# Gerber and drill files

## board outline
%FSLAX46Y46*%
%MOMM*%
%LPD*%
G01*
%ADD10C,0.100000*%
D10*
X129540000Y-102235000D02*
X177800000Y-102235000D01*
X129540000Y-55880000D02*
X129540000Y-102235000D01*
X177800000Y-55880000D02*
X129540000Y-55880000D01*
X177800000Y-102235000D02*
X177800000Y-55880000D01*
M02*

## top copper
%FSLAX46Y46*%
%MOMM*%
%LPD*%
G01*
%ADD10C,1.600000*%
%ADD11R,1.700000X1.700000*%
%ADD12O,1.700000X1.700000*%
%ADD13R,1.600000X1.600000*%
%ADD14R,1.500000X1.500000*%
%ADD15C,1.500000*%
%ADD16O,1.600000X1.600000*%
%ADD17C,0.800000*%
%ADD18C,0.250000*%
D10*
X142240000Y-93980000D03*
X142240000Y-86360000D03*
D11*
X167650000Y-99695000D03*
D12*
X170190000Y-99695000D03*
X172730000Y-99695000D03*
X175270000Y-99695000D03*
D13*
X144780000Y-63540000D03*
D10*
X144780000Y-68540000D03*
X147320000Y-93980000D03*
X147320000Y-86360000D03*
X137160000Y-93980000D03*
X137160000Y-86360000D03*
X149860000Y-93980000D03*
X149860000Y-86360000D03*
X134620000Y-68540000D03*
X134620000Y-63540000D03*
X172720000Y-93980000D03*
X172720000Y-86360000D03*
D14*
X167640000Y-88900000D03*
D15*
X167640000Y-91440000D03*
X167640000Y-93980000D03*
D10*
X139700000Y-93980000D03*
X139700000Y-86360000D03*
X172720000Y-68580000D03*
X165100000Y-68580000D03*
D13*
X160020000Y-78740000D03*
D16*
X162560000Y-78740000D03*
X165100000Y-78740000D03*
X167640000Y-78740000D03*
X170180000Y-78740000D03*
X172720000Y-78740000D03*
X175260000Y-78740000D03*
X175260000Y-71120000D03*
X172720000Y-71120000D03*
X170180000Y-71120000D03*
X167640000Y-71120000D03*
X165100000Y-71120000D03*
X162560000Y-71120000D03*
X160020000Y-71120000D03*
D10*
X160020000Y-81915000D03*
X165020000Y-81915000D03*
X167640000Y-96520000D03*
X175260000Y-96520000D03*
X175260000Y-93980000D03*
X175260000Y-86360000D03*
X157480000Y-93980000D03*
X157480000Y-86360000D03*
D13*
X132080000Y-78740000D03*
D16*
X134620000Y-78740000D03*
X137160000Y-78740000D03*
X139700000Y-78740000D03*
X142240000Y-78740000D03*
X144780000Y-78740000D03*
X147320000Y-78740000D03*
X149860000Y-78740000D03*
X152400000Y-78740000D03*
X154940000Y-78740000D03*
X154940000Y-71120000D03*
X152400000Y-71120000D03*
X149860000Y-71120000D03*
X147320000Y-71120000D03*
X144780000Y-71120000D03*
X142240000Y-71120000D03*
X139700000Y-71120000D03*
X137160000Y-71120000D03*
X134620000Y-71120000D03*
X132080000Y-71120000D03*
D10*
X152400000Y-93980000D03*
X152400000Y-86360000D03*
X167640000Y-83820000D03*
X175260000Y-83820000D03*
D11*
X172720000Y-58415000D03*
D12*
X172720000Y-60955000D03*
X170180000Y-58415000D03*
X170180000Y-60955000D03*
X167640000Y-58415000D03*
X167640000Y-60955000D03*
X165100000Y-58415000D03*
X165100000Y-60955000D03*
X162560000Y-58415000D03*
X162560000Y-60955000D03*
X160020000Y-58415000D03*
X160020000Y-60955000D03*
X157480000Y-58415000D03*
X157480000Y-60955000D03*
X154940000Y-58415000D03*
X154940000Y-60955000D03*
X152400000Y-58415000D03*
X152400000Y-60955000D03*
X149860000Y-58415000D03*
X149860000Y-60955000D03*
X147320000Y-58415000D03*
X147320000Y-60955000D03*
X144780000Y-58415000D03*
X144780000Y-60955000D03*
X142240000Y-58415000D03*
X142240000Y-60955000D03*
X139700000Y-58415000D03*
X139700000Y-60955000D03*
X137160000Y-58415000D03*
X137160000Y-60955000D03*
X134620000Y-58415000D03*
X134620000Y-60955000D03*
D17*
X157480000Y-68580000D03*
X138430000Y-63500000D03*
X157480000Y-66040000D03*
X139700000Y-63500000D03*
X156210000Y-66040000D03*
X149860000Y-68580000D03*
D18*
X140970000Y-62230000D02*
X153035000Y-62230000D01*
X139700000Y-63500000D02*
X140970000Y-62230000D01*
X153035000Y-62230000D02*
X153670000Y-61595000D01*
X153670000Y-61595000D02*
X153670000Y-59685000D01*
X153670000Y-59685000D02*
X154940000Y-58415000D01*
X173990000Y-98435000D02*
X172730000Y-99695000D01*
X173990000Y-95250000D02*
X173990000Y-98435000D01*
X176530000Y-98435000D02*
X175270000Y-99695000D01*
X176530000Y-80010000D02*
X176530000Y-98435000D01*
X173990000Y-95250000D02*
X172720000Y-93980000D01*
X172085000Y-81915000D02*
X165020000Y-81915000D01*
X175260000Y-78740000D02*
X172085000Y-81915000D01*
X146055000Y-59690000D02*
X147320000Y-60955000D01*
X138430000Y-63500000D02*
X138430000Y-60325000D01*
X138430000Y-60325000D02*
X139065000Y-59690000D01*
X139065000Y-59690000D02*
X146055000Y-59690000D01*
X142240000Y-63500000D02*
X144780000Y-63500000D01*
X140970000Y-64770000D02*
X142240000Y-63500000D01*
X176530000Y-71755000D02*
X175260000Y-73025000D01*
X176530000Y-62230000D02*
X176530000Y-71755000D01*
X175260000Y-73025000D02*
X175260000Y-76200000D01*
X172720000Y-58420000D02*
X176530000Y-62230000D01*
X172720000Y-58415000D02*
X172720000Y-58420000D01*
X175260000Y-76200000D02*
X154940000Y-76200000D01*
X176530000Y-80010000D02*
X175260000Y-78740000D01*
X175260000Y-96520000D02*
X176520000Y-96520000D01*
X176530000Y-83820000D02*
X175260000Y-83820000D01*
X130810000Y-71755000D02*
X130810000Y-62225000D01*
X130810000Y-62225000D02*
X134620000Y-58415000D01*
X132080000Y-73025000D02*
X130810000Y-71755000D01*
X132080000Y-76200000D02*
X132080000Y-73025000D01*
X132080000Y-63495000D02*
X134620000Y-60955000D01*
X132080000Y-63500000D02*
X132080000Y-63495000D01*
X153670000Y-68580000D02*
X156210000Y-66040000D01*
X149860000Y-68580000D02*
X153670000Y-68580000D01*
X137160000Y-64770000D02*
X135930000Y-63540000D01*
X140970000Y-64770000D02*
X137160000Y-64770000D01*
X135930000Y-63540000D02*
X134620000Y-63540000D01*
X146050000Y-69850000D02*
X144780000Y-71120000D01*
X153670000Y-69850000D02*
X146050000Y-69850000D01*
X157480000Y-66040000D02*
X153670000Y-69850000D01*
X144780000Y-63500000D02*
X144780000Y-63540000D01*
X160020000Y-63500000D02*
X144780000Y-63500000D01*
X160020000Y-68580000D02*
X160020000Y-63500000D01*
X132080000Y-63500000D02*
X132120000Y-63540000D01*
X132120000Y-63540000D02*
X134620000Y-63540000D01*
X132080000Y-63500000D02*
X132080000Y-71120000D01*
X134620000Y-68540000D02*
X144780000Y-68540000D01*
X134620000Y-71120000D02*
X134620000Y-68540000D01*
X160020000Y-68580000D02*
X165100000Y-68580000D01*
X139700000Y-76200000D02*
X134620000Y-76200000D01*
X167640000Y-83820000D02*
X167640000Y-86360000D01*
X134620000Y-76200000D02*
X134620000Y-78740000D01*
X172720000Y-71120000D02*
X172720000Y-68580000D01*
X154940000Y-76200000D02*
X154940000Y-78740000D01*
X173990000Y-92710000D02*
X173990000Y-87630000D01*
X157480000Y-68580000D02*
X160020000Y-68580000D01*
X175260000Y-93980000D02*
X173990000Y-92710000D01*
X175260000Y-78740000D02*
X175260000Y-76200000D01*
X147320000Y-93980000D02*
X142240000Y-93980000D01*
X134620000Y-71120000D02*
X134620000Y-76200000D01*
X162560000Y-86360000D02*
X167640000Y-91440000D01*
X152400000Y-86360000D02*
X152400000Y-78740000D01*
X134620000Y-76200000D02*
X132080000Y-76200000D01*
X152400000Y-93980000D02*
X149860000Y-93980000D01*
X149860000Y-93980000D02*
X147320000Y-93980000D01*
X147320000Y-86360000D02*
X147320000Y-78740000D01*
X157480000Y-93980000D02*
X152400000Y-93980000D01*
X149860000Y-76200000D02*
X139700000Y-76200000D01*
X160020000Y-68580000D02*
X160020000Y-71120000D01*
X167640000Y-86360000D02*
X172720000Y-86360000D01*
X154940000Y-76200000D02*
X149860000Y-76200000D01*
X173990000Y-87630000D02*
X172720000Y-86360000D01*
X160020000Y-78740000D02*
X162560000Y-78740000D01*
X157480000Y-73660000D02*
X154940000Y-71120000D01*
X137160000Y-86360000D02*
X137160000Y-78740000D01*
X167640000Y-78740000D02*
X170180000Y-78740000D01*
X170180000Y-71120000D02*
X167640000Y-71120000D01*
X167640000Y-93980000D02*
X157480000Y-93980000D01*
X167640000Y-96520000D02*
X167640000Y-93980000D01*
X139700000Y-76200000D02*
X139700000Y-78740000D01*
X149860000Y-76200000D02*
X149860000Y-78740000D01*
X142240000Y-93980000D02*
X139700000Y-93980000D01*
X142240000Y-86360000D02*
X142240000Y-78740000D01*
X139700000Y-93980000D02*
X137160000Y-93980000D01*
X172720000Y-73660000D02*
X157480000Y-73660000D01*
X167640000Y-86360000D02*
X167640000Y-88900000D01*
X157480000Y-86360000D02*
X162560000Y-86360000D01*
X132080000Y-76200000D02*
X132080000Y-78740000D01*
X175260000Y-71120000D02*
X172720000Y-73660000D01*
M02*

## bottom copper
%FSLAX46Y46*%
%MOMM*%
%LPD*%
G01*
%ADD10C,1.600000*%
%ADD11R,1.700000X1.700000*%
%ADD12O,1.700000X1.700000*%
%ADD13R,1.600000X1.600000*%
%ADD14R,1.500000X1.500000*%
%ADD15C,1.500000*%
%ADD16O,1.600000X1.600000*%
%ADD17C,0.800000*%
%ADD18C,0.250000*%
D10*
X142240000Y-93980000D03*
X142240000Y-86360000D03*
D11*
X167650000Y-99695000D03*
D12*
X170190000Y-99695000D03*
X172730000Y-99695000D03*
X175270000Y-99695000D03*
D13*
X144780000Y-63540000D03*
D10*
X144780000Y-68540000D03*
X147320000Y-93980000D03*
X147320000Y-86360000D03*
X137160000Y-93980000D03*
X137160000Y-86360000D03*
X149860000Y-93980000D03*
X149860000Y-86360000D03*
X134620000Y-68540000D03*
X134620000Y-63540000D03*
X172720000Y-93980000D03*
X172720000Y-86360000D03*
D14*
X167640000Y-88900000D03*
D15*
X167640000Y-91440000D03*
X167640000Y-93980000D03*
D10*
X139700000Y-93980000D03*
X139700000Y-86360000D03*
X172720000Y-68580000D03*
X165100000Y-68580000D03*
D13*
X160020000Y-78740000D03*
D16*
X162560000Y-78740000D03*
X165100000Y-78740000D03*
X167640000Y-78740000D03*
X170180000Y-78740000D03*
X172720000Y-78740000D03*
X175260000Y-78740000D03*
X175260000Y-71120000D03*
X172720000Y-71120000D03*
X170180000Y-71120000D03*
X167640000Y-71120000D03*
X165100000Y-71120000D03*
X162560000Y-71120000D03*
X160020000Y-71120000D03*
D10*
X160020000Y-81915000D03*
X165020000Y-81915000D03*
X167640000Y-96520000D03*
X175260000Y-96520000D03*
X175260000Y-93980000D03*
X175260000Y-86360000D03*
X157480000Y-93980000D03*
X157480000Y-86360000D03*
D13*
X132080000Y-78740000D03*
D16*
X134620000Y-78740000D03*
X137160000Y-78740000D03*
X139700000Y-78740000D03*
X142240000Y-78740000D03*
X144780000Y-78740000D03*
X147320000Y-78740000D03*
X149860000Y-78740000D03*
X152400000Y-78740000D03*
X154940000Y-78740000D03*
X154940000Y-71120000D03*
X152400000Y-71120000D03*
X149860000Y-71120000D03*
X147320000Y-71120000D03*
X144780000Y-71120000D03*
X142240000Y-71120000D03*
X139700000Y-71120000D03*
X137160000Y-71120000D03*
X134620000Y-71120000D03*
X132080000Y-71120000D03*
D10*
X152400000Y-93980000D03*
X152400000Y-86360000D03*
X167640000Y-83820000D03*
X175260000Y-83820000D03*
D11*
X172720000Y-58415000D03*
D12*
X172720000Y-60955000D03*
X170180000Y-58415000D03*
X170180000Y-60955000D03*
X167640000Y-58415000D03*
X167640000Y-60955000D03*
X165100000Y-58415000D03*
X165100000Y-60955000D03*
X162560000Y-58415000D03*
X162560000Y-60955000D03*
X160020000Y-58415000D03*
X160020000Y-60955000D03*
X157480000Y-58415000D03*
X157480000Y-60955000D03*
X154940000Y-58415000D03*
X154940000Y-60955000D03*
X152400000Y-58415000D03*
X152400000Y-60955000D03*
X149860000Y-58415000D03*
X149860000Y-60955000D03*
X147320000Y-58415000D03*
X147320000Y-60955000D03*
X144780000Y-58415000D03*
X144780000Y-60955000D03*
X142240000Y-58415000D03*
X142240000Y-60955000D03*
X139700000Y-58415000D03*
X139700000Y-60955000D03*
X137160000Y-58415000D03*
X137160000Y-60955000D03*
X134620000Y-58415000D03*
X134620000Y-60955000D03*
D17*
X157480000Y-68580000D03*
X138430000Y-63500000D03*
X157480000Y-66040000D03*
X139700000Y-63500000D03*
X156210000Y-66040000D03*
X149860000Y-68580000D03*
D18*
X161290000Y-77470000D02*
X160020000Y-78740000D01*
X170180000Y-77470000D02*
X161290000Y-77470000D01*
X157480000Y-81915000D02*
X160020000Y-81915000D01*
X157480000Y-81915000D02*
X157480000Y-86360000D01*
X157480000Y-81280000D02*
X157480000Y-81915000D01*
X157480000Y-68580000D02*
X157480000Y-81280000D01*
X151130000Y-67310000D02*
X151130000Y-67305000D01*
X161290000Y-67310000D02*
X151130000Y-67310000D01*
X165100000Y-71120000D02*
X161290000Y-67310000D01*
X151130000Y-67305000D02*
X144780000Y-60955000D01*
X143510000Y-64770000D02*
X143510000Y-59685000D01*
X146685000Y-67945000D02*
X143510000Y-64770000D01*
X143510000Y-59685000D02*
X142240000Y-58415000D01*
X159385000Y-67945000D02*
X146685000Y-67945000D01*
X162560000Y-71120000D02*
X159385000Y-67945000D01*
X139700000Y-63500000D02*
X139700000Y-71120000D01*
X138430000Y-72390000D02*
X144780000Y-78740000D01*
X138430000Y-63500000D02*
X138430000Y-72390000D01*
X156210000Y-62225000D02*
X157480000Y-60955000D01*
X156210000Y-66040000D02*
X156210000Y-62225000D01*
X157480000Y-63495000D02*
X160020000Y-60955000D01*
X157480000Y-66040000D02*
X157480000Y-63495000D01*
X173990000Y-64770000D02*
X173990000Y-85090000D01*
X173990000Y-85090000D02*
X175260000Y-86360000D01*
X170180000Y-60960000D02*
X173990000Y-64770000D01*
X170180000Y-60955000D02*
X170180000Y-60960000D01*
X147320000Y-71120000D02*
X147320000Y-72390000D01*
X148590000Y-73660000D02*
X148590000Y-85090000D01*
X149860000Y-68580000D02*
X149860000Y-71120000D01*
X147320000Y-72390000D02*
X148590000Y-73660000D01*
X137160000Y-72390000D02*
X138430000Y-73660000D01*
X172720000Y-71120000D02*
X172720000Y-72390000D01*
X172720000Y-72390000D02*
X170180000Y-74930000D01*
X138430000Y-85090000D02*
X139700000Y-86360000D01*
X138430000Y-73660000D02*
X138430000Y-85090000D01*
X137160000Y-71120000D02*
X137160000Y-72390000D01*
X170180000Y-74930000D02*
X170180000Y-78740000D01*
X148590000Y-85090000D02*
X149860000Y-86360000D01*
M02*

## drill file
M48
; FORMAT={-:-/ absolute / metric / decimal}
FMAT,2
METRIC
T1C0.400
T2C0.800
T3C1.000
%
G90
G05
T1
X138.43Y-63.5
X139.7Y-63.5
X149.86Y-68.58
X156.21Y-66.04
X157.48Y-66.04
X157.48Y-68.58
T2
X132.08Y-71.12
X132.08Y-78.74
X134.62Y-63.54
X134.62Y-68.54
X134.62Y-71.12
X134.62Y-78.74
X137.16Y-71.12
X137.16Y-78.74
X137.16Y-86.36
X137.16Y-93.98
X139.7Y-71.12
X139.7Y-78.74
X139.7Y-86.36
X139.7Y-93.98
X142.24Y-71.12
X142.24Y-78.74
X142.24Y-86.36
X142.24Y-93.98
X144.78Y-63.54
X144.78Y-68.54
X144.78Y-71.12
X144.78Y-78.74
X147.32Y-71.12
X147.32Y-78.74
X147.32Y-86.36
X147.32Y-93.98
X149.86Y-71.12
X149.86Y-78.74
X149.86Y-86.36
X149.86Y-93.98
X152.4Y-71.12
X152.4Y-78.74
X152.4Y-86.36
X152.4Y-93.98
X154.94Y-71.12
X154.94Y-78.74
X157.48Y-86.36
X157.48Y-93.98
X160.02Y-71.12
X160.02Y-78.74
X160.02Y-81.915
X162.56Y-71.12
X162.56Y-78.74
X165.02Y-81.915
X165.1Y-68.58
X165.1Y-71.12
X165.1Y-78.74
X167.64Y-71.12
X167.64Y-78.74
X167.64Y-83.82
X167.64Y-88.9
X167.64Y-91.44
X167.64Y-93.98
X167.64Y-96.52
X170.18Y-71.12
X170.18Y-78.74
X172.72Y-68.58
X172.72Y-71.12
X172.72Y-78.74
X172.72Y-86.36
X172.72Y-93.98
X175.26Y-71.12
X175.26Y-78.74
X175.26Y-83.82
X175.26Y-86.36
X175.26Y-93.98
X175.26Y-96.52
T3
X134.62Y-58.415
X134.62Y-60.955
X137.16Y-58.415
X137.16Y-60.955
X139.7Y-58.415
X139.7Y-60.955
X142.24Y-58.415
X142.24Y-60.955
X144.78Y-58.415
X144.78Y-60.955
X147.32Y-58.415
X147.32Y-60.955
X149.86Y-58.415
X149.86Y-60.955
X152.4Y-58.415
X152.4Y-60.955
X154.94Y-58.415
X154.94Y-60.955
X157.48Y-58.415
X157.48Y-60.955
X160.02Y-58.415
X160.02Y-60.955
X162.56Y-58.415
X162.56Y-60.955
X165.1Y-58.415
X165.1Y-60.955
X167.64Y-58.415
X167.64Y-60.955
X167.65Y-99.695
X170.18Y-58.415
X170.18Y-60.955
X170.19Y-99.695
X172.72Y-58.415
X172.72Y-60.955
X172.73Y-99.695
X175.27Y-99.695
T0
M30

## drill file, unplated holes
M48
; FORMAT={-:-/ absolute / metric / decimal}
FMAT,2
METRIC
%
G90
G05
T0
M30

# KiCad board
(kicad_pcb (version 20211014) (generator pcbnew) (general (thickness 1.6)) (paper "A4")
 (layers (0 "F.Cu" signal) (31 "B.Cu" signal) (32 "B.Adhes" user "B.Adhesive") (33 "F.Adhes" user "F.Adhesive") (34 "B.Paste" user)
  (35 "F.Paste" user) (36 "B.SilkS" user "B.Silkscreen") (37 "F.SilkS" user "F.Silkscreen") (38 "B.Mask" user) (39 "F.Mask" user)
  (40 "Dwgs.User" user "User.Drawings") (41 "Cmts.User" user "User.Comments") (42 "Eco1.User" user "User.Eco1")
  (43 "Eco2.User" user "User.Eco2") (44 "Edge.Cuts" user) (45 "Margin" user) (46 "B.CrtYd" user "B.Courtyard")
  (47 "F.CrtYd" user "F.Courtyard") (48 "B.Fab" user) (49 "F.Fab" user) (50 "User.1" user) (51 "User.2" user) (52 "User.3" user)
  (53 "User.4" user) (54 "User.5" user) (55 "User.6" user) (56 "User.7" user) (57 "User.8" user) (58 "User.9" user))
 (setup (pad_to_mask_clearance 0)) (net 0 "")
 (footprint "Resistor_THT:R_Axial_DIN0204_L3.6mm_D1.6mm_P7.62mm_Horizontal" (layer "F.Cu") (at 142.24 93.98 90)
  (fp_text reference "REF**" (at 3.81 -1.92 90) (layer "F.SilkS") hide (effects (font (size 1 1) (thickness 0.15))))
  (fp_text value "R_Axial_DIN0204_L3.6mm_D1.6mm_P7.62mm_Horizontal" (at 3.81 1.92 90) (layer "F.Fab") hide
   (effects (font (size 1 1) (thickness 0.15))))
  (pad "1" thru_hole circle (at 0 0 90) (size 1.6 1.6) (drill 0.8) (layers *.Cu *.Mask))
  (pad "2" thru_hole circle (at 7.62 0 90) (size 1.6 1.6) (drill 0.8) (layers *.Cu *.Mask)))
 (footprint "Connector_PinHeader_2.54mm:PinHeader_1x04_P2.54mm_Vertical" (layer "F.Cu") (at 167.65 99.695 90)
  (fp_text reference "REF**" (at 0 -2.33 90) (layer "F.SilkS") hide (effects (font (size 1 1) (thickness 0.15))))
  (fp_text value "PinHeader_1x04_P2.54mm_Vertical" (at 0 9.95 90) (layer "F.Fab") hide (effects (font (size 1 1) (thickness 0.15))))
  (pad "1" thru_hole rect (at 0 0 90) (size 1.7 1.7) (drill 1) (layers *.Cu *.Mask))
  (pad "2" thru_hole oval (at 0 2.54 90) (size 1.7 1.7) (drill 1) (layers *.Cu *.Mask))
  (pad "3" thru_hole oval (at 0 5.08 90) (size 1.7 1.7) (drill 1) (layers *.Cu *.Mask))
  (pad "4" thru_hole oval (at 0 7.62 90) (size 1.7 1.7) (drill 1) (layers *.Cu *.Mask)))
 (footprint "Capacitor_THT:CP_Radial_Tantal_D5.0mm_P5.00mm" (layer "F.Cu") (at 144.78 63.54 -90)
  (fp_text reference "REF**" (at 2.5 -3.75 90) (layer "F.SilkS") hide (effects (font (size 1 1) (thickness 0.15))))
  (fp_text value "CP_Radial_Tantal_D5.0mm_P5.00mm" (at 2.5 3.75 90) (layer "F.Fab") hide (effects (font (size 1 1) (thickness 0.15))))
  (pad "1" thru_hole rect (at 0 0 270) (size 1.6 1.6) (drill 0.8) (layers *.Cu *.Mask))
  (pad "2" thru_hole circle (at 5 0 270) (size 1.6 1.6) (drill 0.8) (layers *.Cu *.Mask)))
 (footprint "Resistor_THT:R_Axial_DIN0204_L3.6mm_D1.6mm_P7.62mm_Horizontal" (layer "F.Cu") (at 147.32 93.98 90)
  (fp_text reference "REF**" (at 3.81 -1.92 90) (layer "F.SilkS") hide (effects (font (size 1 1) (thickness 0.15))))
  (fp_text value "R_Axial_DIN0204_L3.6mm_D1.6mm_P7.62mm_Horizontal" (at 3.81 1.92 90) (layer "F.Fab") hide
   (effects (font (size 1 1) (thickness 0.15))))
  (pad "1" thru_hole circle (at 0 0 90) (size 1.6 1.6) (drill 0.8) (layers *.Cu *.Mask))
  (pad "2" thru_hole circle (at 7.62 0 90) (size 1.6 1.6) (drill 0.8) (layers *.Cu *.Mask)))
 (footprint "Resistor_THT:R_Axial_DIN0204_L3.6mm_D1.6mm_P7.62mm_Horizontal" (layer "F.Cu") (at 137.16 93.98 90)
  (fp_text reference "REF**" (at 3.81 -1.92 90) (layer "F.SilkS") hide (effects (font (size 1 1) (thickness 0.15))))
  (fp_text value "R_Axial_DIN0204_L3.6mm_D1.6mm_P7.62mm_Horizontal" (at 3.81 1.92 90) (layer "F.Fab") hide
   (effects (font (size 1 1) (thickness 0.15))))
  (pad "1" thru_hole circle (at 0 0 90) (size 1.6 1.6) (drill 0.8) (layers *.Cu *.Mask))
  (pad "2" thru_hole circle (at 7.62 0 90) (size 1.6 1.6) (drill 0.8) (layers *.Cu *.Mask)))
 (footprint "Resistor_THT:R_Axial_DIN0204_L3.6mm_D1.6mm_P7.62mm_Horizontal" (layer "F.Cu") (at 149.86 93.98 90)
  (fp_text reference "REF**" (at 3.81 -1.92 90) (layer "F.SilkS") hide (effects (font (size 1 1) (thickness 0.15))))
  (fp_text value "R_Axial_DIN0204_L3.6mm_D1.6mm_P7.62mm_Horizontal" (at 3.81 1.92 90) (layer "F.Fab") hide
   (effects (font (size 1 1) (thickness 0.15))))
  (pad "1" thru_hole circle (at 0 0 90) (size 1.6 1.6) (drill 0.8) (layers *.Cu *.Mask))
  (pad "2" thru_hole circle (at 7.62 0 90) (size 1.6 1.6) (drill 0.8) (layers *.Cu *.Mask)))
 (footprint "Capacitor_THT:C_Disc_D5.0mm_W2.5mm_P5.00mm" (layer "F.Cu") (at 134.62 68.54 90)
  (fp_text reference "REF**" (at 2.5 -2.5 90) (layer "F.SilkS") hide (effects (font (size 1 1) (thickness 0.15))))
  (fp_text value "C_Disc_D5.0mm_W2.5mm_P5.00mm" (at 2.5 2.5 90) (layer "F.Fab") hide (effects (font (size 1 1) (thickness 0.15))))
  (pad "1" thru_hole circle (at 0 0 90) (size 1.6 1.6) (drill 0.8) (layers *.Cu *.Mask))
  (pad "2" thru_hole circle (at 5 0 90) (size 1.6 1.6) (drill 0.8) (layers *.Cu *.Mask)))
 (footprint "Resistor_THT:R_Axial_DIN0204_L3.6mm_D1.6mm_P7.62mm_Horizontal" (layer "F.Cu") (at 172.72 93.98 90)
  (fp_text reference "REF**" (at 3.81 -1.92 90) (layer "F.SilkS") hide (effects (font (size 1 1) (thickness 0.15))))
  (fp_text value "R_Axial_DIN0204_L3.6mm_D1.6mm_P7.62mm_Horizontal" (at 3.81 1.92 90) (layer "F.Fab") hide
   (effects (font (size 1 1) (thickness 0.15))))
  (pad "1" thru_hole circle (at 0 0 90) (size 1.6 1.6) (drill 0.8) (layers *.Cu *.Mask))
  (pad "2" thru_hole circle (at 7.62 0 90) (size 1.6 1.6) (drill 0.8) (layers *.Cu *.Mask)))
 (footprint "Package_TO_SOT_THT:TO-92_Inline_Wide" (layer "F.Cu") (at 167.64 88.9 -90)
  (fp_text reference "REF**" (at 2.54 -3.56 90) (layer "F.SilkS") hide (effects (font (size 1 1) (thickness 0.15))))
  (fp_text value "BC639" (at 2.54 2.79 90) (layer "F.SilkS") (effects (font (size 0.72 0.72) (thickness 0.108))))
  (pad "1" thru_hole rect (at 0 0 270) (size 1.5 1.5) (drill 0.8) (layers *.Cu *.Mask))
  (pad "2" thru_hole circle (at 2.54 0 270) (size 1.5 1.5) (drill 0.8) (layers *.Cu *.Mask))
  (pad "3" thru_hole circle (at 5.08 0 270) (size 1.5 1.5) (drill 0.8) (layers *.Cu *.Mask)))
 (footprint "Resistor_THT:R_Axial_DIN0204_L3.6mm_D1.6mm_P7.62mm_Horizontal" (layer "F.Cu") (at 139.7 93.98 90)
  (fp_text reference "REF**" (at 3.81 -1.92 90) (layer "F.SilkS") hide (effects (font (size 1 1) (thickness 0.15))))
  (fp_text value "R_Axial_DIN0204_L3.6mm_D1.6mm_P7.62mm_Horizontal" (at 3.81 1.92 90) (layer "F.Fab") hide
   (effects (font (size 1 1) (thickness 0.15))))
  (pad "1" thru_hole circle (at 0 0 90) (size 1.6 1.6) (drill 0.8) (layers *.Cu *.Mask))
  (pad "2" thru_hole circle (at 7.62 0 90) (size 1.6 1.6) (drill 0.8) (layers *.Cu *.Mask)))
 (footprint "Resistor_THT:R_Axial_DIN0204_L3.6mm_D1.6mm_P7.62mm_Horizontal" (layer "F.Cu") (at 172.72 68.58 180)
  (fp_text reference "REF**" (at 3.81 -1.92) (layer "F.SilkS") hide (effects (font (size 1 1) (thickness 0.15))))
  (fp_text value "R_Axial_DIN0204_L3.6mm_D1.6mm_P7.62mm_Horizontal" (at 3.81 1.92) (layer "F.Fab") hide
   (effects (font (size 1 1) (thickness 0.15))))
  (pad "1" thru_hole circle (at 0 0 180) (size 1.6 1.6) (drill 0.8) (layers *.Cu *.Mask))
  (pad "2" thru_hole circle (at 7.62 0 180) (size 1.6 1.6) (drill 0.8) (layers *.Cu *.Mask)))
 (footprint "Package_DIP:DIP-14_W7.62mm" (layer "F.Cu") (at 160.02 78.74 90)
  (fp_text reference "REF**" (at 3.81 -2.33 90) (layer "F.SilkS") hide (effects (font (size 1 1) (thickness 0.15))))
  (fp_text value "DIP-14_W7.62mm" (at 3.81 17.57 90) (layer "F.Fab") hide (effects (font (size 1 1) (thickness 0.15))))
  (pad "1" thru_hole rect (at 0 0 90) (size 1.6 1.6) (drill 0.8) (layers *.Cu *.Mask))
  (pad "2" thru_hole oval (at 0 2.54 90) (size 1.6 1.6) (drill 0.8) (layers *.Cu *.Mask))
  (pad "3" thru_hole oval (at 0 5.08 90) (size 1.6 1.6) (drill 0.8) (layers *.Cu *.Mask))
  (pad "4" thru_hole oval (at 0 7.62 90) (size 1.6 1.6) (drill 0.8) (layers *.Cu *.Mask))
  (pad "5" thru_hole oval (at 0 10.16 90) (size 1.6 1.6) (drill 0.8) (layers *.Cu *.Mask))
  (pad "6" thru_hole oval (at 0 12.7 90) (size 1.6 1.6) (drill 0.8) (layers *.Cu *.Mask))
  (pad "7" thru_hole oval (at 0 15.24 90) (size 1.6 1.6) (drill 0.8) (layers *.Cu *.Mask))
  (pad "8" thru_hole oval (at 7.62 15.24 90) (size 1.6 1.6) (drill 0.8) (layers *.Cu *.Mask))
  (pad "9" thru_hole oval (at 7.62 12.7 90) (size 1.6 1.6) (drill 0.8) (layers *.Cu *.Mask))
  (pad "10" thru_hole oval (at 7.62 10.16 90) (size 1.6 1.6) (drill 0.8) (layers *.Cu *.Mask))
  (pad "11" thru_hole oval (at 7.62 7.62 90) (size 1.6 1.6) (drill 0.8) (layers *.Cu *.Mask))
  (pad "12" thru_hole oval (at 7.62 5.08 90) (size 1.6 1.6) (drill 0.8) (layers *.Cu *.Mask))
  (pad "13" thru_hole oval (at 7.62 2.54 90) (size 1.6 1.6) (drill 0.8) (layers *.Cu *.Mask))
  (pad "14" thru_hole oval (at 7.62 0 90) (size 1.6 1.6) (drill 0.8) (layers *.Cu *.Mask)))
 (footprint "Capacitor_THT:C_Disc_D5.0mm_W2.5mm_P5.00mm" (layer "F.Cu") (at 160.02 81.915)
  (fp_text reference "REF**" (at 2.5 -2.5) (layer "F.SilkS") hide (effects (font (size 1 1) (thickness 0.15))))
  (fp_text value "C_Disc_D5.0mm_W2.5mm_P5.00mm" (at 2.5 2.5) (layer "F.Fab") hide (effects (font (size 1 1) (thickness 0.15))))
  (pad "1" thru_hole circle (at 0 0) (size 1.6 1.6) (drill 0.8) (layers *.Cu *.Mask))
  (pad "2" thru_hole circle (at 5 0) (size 1.6 1.6) (drill 0.8) (layers *.Cu *.Mask)))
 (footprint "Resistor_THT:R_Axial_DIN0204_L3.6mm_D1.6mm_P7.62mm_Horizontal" (layer "F.Cu") (at 167.64 96.52)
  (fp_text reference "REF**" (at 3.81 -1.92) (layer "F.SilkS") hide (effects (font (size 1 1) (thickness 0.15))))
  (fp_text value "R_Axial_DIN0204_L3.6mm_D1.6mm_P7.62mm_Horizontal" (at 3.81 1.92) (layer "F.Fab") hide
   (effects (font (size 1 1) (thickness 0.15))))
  (pad "1" thru_hole circle (at 0 0) (size 1.6 1.6) (drill 0.8) (layers *.Cu *.Mask))
  (pad "2" thru_hole circle (at 7.62 0) (size 1.6 1.6) (drill 0.8) (layers *.Cu *.Mask)))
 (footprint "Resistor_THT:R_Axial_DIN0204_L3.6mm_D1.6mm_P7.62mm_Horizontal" (layer "F.Cu") (at 175.26 93.98 90)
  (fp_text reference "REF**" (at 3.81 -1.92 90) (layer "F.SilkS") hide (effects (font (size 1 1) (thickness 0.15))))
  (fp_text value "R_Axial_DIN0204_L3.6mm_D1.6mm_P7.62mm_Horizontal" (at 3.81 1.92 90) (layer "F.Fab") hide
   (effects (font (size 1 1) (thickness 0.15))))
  (pad "1" thru_hole circle (at 0 0 90) (size 1.6 1.6) (drill 0.8) (layers *.Cu *.Mask))
  (pad "2" thru_hole circle (at 7.62 0 90) (size 1.6 1.6) (drill 0.8) (layers *.Cu *.Mask)))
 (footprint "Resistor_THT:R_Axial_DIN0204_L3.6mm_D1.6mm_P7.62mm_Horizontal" (layer "F.Cu") (at 157.48 93.98 90)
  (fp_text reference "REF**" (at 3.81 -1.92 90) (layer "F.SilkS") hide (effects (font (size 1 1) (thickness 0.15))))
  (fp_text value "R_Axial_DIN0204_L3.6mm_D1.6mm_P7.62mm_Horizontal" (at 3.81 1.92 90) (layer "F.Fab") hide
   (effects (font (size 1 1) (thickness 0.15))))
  (pad "1" thru_hole circle (at 0 0 90) (size 1.6 1.6) (drill 0.8) (layers *.Cu *.Mask))
  (pad "2" thru_hole circle (at 7.62 0 90) (size 1.6 1.6) (drill 0.8) (layers *.Cu *.Mask)))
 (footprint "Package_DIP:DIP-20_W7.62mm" (layer "F.Cu") (at 132.08 78.74 90)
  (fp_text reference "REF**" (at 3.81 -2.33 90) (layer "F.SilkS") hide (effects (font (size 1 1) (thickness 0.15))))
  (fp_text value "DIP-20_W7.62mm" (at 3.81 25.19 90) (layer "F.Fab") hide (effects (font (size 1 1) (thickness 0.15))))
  (pad "1" thru_hole rect (at 0 0 90) (size 1.6 1.6) (drill 0.8) (layers *.Cu *.Mask))
  (pad "2" thru_hole oval (at 0 2.54 90) (size 1.6 1.6) (drill 0.8) (layers *.Cu *.Mask))
  (pad "3" thru_hole oval (at 0 5.08 90) (size 1.6 1.6) (drill 0.8) (layers *.Cu *.Mask))
  (pad "4" thru_hole oval (at 0 7.62 90) (size 1.6 1.6) (drill 0.8) (layers *.Cu *.Mask))
  (pad "5" thru_hole oval (at 0 10.16 90) (size 1.6 1.6) (drill 0.8) (layers *.Cu *.Mask))
  (pad "6" thru_hole oval (at 0 12.7 90) (size 1.6 1.6) (drill 0.8) (layers *.Cu *.Mask))
  (pad "7" thru_hole oval (at 0 15.24 90) (size 1.6 1.6) (drill 0.8) (layers *.Cu *.Mask))
  (pad "8" thru_hole oval (at 0 17.78 90) (size 1.6 1.6) (drill 0.8) (layers *.Cu *.Mask))
  (pad "9" thru_hole oval (at 0 20.32 90) (size 1.6 1.6) (drill 0.8) (layers *.Cu *.Mask))
  (pad "10" thru_hole oval (at 0 22.86 90) (size 1.6 1.6) (drill 0.8) (layers *.Cu *.Mask))
  (pad "11" thru_hole oval (at 7.62 22.86 90) (size 1.6 1.6) (drill 0.8) (layers *.Cu *.Mask))
  (pad "12" thru_hole oval (at 7.62 20.32 90) (size 1.6 1.6) (drill 0.8) (layers *.Cu *.Mask))
  (pad "13" thru_hole oval (at 7.62 17.78 90) (size 1.6 1.6) (drill 0.8) (layers *.Cu *.Mask))
  (pad "14" thru_hole oval (at 7.62 15.24 90) (size 1.6 1.6) (drill 0.8) (layers *.Cu *.Mask))
  (pad "15" thru_hole oval (at 7.62 12.7 90) (size 1.6 1.6) (drill 0.8) (layers *.Cu *.Mask))
  (pad "16" thru_hole oval (at 7.62 10.16 90) (size 1.6 1.6) (drill 0.8) (layers *.Cu *.Mask))
  (pad "17" thru_hole oval (at 7.62 7.62 90) (size 1.6 1.6) (drill 0.8) (layers *.Cu *.Mask))
  (pad "18" thru_hole oval (at 7.62 5.08 90) (size 1.6 1.6) (drill 0.8) (layers *.Cu *.Mask))
  (pad "19" thru_hole oval (at 7.62 2.54 90) (size 1.6 1.6) (drill 0.8) (layers *.Cu *.Mask))
  (pad "20" thru_hole oval (at 7.62 0 90) (size 1.6 1.6) (drill 0.8) (layers *.Cu *.Mask)))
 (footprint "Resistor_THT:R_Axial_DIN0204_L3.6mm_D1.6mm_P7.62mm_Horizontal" (layer "F.Cu") (at 152.4 93.98 90)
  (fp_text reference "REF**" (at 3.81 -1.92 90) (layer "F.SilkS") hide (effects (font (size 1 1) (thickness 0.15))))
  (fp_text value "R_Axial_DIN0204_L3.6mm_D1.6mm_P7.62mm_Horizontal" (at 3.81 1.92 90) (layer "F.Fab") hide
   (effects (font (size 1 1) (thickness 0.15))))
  (pad "1" thru_hole circle (at 0 0 90) (size 1.6 1.6) (drill 0.8) (layers *.Cu *.Mask))
  (pad "2" thru_hole circle (at 7.62 0 90) (size 1.6 1.6) (drill 0.8) (layers *.Cu *.Mask)))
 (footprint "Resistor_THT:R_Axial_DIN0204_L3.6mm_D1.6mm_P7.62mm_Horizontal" (layer "F.Cu") (at 167.64 83.82)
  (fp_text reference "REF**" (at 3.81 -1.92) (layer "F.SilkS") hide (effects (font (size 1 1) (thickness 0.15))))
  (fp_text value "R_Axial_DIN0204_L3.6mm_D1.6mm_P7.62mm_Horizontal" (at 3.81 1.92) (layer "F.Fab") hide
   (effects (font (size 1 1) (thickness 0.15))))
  (pad "1" thru_hole circle (at 0 0) (size 1.6 1.6) (drill 0.8) (layers *.Cu *.Mask))
  (pad "2" thru_hole circle (at 7.62 0) (size 1.6 1.6) (drill 0.8) (layers *.Cu *.Mask)))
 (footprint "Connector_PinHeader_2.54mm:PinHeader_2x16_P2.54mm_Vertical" (layer "B.Cu") (at 172.72 61.795 90)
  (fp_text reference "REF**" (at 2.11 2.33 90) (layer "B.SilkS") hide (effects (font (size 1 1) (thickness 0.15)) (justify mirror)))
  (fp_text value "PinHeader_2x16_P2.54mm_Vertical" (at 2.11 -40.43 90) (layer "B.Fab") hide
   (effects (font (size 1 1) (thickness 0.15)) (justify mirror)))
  (pad "1" thru_hole rect (at 3.38 0 90) (size 1.7 1.7) (drill 1) (layers *.Cu *.Mask))
  (pad "2" thru_hole oval (at 0.84 0 90) (size 1.7 1.7) (drill 1) (layers *.Cu *.Mask))
  (pad "3" thru_hole oval (at 3.38 -2.54 90) (size 1.7 1.7) (drill 1) (layers *.Cu *.Mask))
  (pad "4" thru_hole oval (at 0.84 -2.54 90) (size 1.7 1.7) (drill 1) (layers *.Cu *.Mask))
  (pad "5" thru_hole oval (at 3.38 -5.08 90) (size 1.7 1.7) (drill 1) (layers *.Cu *.Mask))
  (pad "6" thru_hole oval (at 0.84 -5.08 90) (size 1.7 1.7) (drill 1) (layers *.Cu *.Mask))
  (pad "7" thru_hole oval (at 3.38 -7.62 90) (size 1.7 1.7) (drill 1) (layers *.Cu *.Mask))
  (pad "8" thru_hole oval (at 0.84 -7.62 90) (size 1.7 1.7) (drill 1) (layers *.Cu *.Mask))
  (pad "9" thru_hole oval (at 3.38 -10.16 90) (size 1.7 1.7) (drill 1) (layers *.Cu *.Mask))
  (pad "10" thru_hole oval (at 0.84 -10.16 90) (size 1.7 1.7) (drill 1) (layers *.Cu *.Mask))
  (pad "11" thru_hole oval (at 3.38 -12.7 90) (size 1.7 1.7) (drill 1) (layers *.Cu *.Mask))
  (pad "12" thru_hole oval (at 0.84 -12.7 90) (size 1.7 1.7) (drill 1) (layers *.Cu *.Mask))
  (pad "13" thru_hole oval (at 3.38 -15.24 90) (size 1.7 1.7) (drill 1) (layers *.Cu *.Mask))
  (pad "14" thru_hole oval (at 0.84 -15.24 90) (size 1.7 1.7) (drill 1) (layers *.Cu *.Mask))
  (pad "15" thru_hole oval (at 3.38 -17.78 90) (size 1.7 1.7) (drill 1) (layers *.Cu *.Mask))
  (pad "16" thru_hole oval (at 0.84 -17.78 90) (size 1.7 1.7) (drill 1) (layers *.Cu *.Mask))
  (pad "17" thru_hole oval (at 3.38 -20.32 90) (size 1.7 1.7) (drill 1) (layers *.Cu *.Mask))
  (pad "18" thru_hole oval (at 0.84 -20.32 90) (size 1.7 1.7) (drill 1) (layers *.Cu *.Mask))
  (pad "19" thru_hole oval (at 3.38 -22.86 90) (size 1.7 1.7) (drill 1) (layers *.Cu *.Mask))
  (pad "20" thru_hole oval (at 0.84 -22.86 90) (size 1.7 1.7) (drill 1) (layers *.Cu *.Mask))
  (pad "21" thru_hole oval (at 3.38 -25.4 90) (size 1.7 1.7) (drill 1) (layers *.Cu *.Mask))
  (pad "22" thru_hole oval (at 0.84 -25.4 90) (size 1.7 1.7) (drill 1) (layers *.Cu *.Mask))
  (pad "23" thru_hole oval (at 3.38 -27.94 90) (size 1.7 1.7) (drill 1) (layers *.Cu *.Mask))
  (pad "24" thru_hole oval (at 0.84 -27.94 90) (size 1.7 1.7) (drill 1) (layers *.Cu *.Mask))
  (pad "25" thru_hole oval (at 3.38 -30.48 90) (size 1.7 1.7) (drill 1) (layers *.Cu *.Mask))
  (pad "26" thru_hole oval (at 0.84 -30.48 90) (size 1.7 1.7) (drill 1) (layers *.Cu *.Mask))
  (pad "27" thru_hole oval (at 3.38 -33.02 90) (size 1.7 1.7) (drill 1) (layers *.Cu *.Mask))
  (pad "28" thru_hole oval (at 0.84 -33.02 90) (size 1.7 1.7) (drill 1) (layers *.Cu *.Mask))
  (pad "29" thru_hole oval (at 3.38 -35.56 90) (size 1.7 1.7) (drill 1) (layers *.Cu *.Mask))
  (pad "30" thru_hole oval (at 0.84 -35.56 90) (size 1.7 1.7) (drill 1) (layers *.Cu *.Mask))
  (pad "31" thru_hole oval (at 3.38 -38.1 90) (size 1.7 1.7) (drill 1) (layers *.Cu *.Mask))
  (pad "32" thru_hole oval (at 0.84 -38.1 90) (size 1.7 1.7) (drill 1) (layers *.Cu *.Mask)))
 (gr_line (start 177.8 102.235) (end 177.8 55.88) (layer "Edge.Cuts") (width 0.1))
 (gr_line (start 177.8 55.88) (end 129.54 55.88) (layer "Edge.Cuts") (width 0.1))
 (gr_line (start 129.54 102.235) (end 177.8 102.235) (layer "Edge.Cuts") (width 0.1))
 (gr_line (start 129.54 55.88) (end 129.54 102.235) (layer "Edge.Cuts") (width 0.1))
 (segment (start 132.08 63.5) (end 132.12 63.54) (width 0.25) (layer "F.Cu") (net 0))
 (segment (start 173.99 95.25) (end 172.72 93.98) (width 0.25) (layer "F.Cu") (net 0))
 (segment (start 153.67 61.595) (end 153.67 59.685) (width 0.25) (layer "F.Cu") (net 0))
 (segment (start 139.7 76.2) (end 134.62 76.2) (width 0.25) (layer "F.Cu") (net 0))
 (segment (start 167.64 83.82) (end 167.64 86.36) (width 0.25) (layer "F.Cu") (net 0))
 (segment (start 134.62 76.2) (end 134.62 78.74) (width 0.25) (layer "F.Cu") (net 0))
 (segment (start 157.48 66.04) (end 153.67 69.85) (width 0.25) (layer "F.Cu") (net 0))
 (segment (start 160.02 63.5) (end 144.78 63.5) (width 0.25) (layer "F.Cu") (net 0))
 (segment (start 172.72 71.12) (end 172.72 68.58) (width 0.25) (layer "F.Cu") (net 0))
 (segment (start 132.08 63.5) (end 132.08 63.495) (width 0.25) (layer "F.Cu") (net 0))
 (segment (start 132.12 63.54) (end 134.62 63.54) (width 0.25) (layer "F.Cu") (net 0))
 (segment (start 173.99 98.435) (end 172.73 99.695) (width 0.25) (layer "F.Cu") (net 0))
 (segment (start 175.26 96.52) (end 176.52 96.52) (width 0.25) (layer "F.Cu") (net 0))
 (segment (start 154.94 76.2) (end 154.94 78.74) (width 0.25) (layer "F.Cu") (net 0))
 (segment (start 173.99 92.71) (end 173.99 87.63) (width 0.25) (layer "F.Cu") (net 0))
 (segment (start 176.53 80.01) (end 176.53 98.435) (width 0.25) (layer "F.Cu") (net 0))
 (segment (start 149.86 68.58) (end 153.67 68.58) (width 0.25) (layer "F.Cu") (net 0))
 (segment (start 157.48 68.58) (end 160.02 68.58) (width 0.25) (layer "F.Cu") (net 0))
 (segment (start 175.26 93.98) (end 173.99 92.71) (width 0.25) (layer "F.Cu") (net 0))
 (segment (start 176.53 98.435) (end 175.27 99.695) (width 0.25) (layer "F.Cu") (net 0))
 (segment (start 146.055 59.69) (end 147.32 60.955) (width 0.25) (layer "F.Cu") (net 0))
 (segment (start 130.81 62.225) (end 134.62 58.415) (width 0.25) (layer "F.Cu") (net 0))
 (segment (start 175.26 78.74) (end 175.26 76.2) (width 0.25) (layer "F.Cu") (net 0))
 (segment (start 147.32 93.98) (end 142.24 93.98) (width 0.25) (layer "F.Cu") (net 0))
 (segment (start 139.7 63.5) (end 140.97 62.23) (width 0.25) (layer "F.Cu") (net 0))
 (segment (start 146.05 69.85) (end 144.78 71.12) (width 0.25) (layer "F.Cu") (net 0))
 (segment (start 176.53 80.01) (end 175.26 78.74) (width 0.25) (layer "F.Cu") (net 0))
 (segment (start 134.62 71.12) (end 134.62 76.2) (width 0.25) (layer "F.Cu") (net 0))
 (segment (start 162.56 86.36) (end 167.64 91.44) (width 0.25) (layer "F.Cu") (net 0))
 (segment (start 152.4 86.36) (end 152.4 78.74) (width 0.25) (layer "F.Cu") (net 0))
 (segment (start 160.02 68.58) (end 160.02 63.5) (width 0.25) (layer "F.Cu") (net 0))
 (segment (start 153.035 62.23) (end 153.67 61.595) (width 0.25) (layer "F.Cu") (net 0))
 (segment (start 137.16 64.77) (end 135.93 63.54) (width 0.25) (layer "F.Cu") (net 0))
 (segment (start 134.62 76.2) (end 132.08 76.2) (width 0.25) (layer "F.Cu") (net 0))
 (segment (start 172.72 58.42) (end 176.53 62.23) (width 0.25) (layer "F.Cu") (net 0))
 (segment (start 152.4 93.98) (end 149.86 93.98) (width 0.25) (layer "F.Cu") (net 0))
 (segment (start 149.86 93.98) (end 147.32 93.98) (width 0.25) (layer "F.Cu") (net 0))
 (segment (start 140.97 64.77) (end 142.24 63.5) (width 0.25) (layer "F.Cu") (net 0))
 (segment (start 172.72 58.415) (end 172.72 58.42) (width 0.25) (layer "F.Cu") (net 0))
 (segment (start 153.67 68.58) (end 156.21 66.04) (width 0.25) (layer "F.Cu") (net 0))
 (segment (start 140.97 62.23) (end 153.035 62.23) (width 0.25) (layer "F.Cu") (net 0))
 (segment (start 147.32 86.36) (end 147.32 78.74) (width 0.25) (layer "F.Cu") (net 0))
 (segment (start 157.48 93.98) (end 152.4 93.98) (width 0.25) (layer "F.Cu") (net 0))
 (segment (start 175.26 78.74) (end 172.085 81.915) (width 0.25) (layer "F.Cu") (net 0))
 (segment (start 149.86 76.2) (end 139.7 76.2) (width 0.25) (layer "F.Cu") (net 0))
 (segment (start 132.08 63.495) (end 134.62 60.955) (width 0.25) (layer "F.Cu") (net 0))
 (segment (start 160.02 68.58) (end 160.02 71.12) (width 0.25) (layer "F.Cu") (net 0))
 (segment (start 167.64 86.36) (end 172.72 86.36) (width 0.25) (layer "F.Cu") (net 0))
 (segment (start 172.085 81.915) (end 165.02 81.915) (width 0.25) (layer "F.Cu") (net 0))
 (segment (start 154.94 76.2) (end 149.86 76.2) (width 0.25) (layer "F.Cu") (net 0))
 (segment (start 173.99 87.63) (end 172.72 86.36) (width 0.25) (layer "F.Cu") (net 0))
 (segment (start 142.24 63.5) (end 144.78 63.5) (width 0.25) (layer "F.Cu") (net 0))
 (segment (start 160.02 78.74) (end 162.56 78.74) (width 0.25) (layer "F.Cu") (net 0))
 (segment (start 157.48 73.66) (end 154.94 71.12) (width 0.25) (layer "F.Cu") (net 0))
 (segment (start 137.16 86.36) (end 137.16 78.74) (width 0.25) (layer "F.Cu") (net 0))
 (segment (start 153.67 59.685) (end 154.94 58.415) (width 0.25) (layer "F.Cu") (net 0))
 (segment (start 132.08 76.2) (end 132.08 73.025) (width 0.25) (layer "F.Cu") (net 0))
 (segment (start 160.02 68.58) (end 165.1 68.58) (width 0.25) (layer "F.Cu") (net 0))
 (segment (start 132.08 63.5) (end 132.08 71.12) (width 0.25) (layer "F.Cu") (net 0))
 (segment (start 167.64 78.74) (end 170.18 78.74) (width 0.25) (layer "F.Cu") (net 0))
 (segment (start 140.97 64.77) (end 137.16 64.77) (width 0.25) (layer "F.Cu") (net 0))
 (segment (start 170.18 71.12) (end 167.64 71.12) (width 0.25) (layer "F.Cu") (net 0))
 (segment (start 135.93 63.54) (end 134.62 63.54) (width 0.25) (layer "F.Cu") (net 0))
 (segment (start 167.64 93.98) (end 157.48 93.98) (width 0.25) (layer "F.Cu") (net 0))
 (segment (start 167.64 96.52) (end 167.64 93.98) (width 0.25) (layer "F.Cu") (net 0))
 (segment (start 173.99 95.25) (end 173.99 98.435) (width 0.25) (layer "F.Cu") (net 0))
 (segment (start 139.7 76.2) (end 139.7 78.74) (width 0.25) (layer "F.Cu") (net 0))
 (segment (start 176.53 62.23) (end 176.53 71.755) (width 0.25) (layer "F.Cu") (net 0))
 (segment (start 149.86 76.2) (end 149.86 78.74) (width 0.25) (layer "F.Cu") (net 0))
 (segment (start 142.24 93.98) (end 139.7 93.98) (width 0.25) (layer "F.Cu") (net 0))
 (segment (start 130.81 71.755) (end 130.81 62.225) (width 0.25) (layer "F.Cu") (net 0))
 (segment (start 142.24 86.36) (end 142.24 78.74) (width 0.25) (layer "F.Cu") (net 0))
 (segment (start 138.43 63.5) (end 138.43 60.325) (width 0.25) (layer "F.Cu") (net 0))
 (segment (start 176.53 83.82) (end 175.26 83.82) (width 0.25) (layer "F.Cu") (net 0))
 (segment (start 139.7 93.98) (end 137.16 93.98) (width 0.25) (layer "F.Cu") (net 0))
 (segment (start 176.53 71.755) (end 175.26 73.025) (width 0.25) (layer "F.Cu") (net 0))
 (segment (start 132.08 73.025) (end 130.81 71.755) (width 0.25) (layer "F.Cu") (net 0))
 (segment (start 172.72 73.66) (end 157.48 73.66) (width 0.25) (layer "F.Cu") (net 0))
 (segment (start 139.065 59.69) (end 146.055 59.69) (width 0.25) (layer "F.Cu") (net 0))
 (segment (start 134.62 68.54) (end 144.78 68.54) (width 0.25) (layer "F.Cu") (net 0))
 (segment (start 167.64 86.36) (end 167.64 88.9) (width 0.25) (layer "F.Cu") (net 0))
 (segment (start 138.43 60.325) (end 139.065 59.69) (width 0.25) (layer "F.Cu") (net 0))
 (segment (start 134.62 71.12) (end 134.62 68.54) (width 0.25) (layer "F.Cu") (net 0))
 (segment (start 157.48 86.36) (end 162.56 86.36) (width 0.25) (layer "F.Cu") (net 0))
 (segment (start 132.08 76.2) (end 132.08 78.74) (width 0.25) (layer "F.Cu") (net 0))
 (segment (start 175.26 76.2) (end 154.94 76.2) (width 0.25) (layer "F.Cu") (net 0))
 (segment (start 144.78 63.5) (end 144.78 63.54) (width 0.25) (layer "F.Cu") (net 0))
 (segment (start 153.67 69.85) (end 146.05 69.85) (width 0.25) (layer "F.Cu") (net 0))
 (segment (start 175.26 71.12) (end 172.72 73.66) (width 0.25) (layer "F.Cu") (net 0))
 (segment (start 175.26 73.025) (end 175.26 76.2) (width 0.25) (layer "F.Cu") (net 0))
 (via (at 157.48 68.58) (size 0.8) (drill 0.4) (layers "F.Cu" "B.Cu") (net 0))
 (via (at 138.43 63.5) (size 0.8) (drill 0.4) (layers "F.Cu" "B.Cu") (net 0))
 (via (at 157.48 66.04) (size 0.8) (drill 0.4) (layers "F.Cu" "B.Cu") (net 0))
 (via (at 139.7 63.5) (size 0.8) (drill 0.4) (layers "F.Cu" "B.Cu") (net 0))
 (via (at 156.21 66.04) (size 0.8) (drill 0.4) (layers "F.Cu" "B.Cu") (free) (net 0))
 (via (at 149.86 68.58) (size 0.8) (drill 0.4) (layers "F.Cu" "B.Cu") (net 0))
 (segment (start 143.51 64.77) (end 143.51 59.685) (width 0.25) (layer "B.Cu") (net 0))
 (segment (start 157.48 81.28) (end 157.48 81.915) (width 0.25) (layer "B.Cu") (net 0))
 (segment (start 147.32 71.12) (end 147.32 72.39) (width 0.25) (layer "B.Cu") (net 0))
 (segment (start 157.48 63.495) (end 160.02 60.955) (width 0.25) (layer "B.Cu") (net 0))
 (segment (start 148.59 73.66) (end 148.59 85.09) (width 0.25) (layer "B.Cu") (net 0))
 (segment (start 149.86 68.58) (end 149.86 71.12) (width 0.25) (layer "B.Cu") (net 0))
 (segment (start 170.18 60.96) (end 173.99 64.77) (width 0.25) (layer "B.Cu") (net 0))
 (segment (start 159.385 67.945) (end 146.685 67.945) (width 0.25) (layer "B.Cu") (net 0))
 (segment (start 138.43 63.5) (end 138.43 72.39) (width 0.25) (layer "B.Cu") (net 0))
 (segment (start 157.48 81.915) (end 160.02 81.915) (width 0.25) (layer "B.Cu") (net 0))
 (segment (start 147.32 72.39) (end 148.59 73.66) (width 0.25) (layer "B.Cu") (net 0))
 (segment (start 161.29 77.47) (end 160.02 78.74) (width 0.25) (layer "B.Cu") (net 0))
 (segment (start 146.685 67.945) (end 143.51 64.77) (width 0.25) (layer "B.Cu") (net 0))
 (segment (start 156.21 62.225) (end 157.48 60.955) (width 0.25) (layer "B.Cu") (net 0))
 (segment (start 156.21 66.04) (end 156.21 62.225) (width 0.25) (layer "B.Cu") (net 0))
 (segment (start 151.13 67.305) (end 144.78 60.955) (width 0.25) (layer "B.Cu") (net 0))
 (segment (start 170.18 77.47) (end 161.29 77.47) (width 0.25) (layer "B.Cu") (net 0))
 (segment (start 137.16 72.39) (end 138.43 73.66) (width 0.25) (layer "B.Cu") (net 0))
 (segment (start 138.43 72.39) (end 144.78 78.74) (width 0.25) (layer "B.Cu") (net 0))
 (segment (start 143.51 59.685) (end 142.24 58.415) (width 0.25) (layer "B.Cu") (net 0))
 (segment (start 172.72 71.12) (end 172.72 72.39) (width 0.25) (layer "B.Cu") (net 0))
 (segment (start 151.13 67.31) (end 151.13 67.305) (width 0.25) (layer "B.Cu") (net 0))
 (segment (start 161.29 67.31) (end 151.13 67.31) (width 0.25) (layer "B.Cu") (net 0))
 (segment (start 173.99 64.77) (end 173.99 85.09) (width 0.25) (layer "B.Cu") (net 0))
 (segment (start 139.7 63.5) (end 139.7 71.12) (width 0.25) (layer "B.Cu") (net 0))
 (segment (start 172.72 72.39) (end 170.18 74.93) (width 0.25) (layer "B.Cu") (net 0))
 (segment (start 138.43 85.09) (end 139.7 86.36) (width 0.25) (layer "B.Cu") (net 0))
 (segment (start 138.43 73.66) (end 138.43 85.09) (width 0.25) (layer "B.Cu") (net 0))
 (segment (start 173.99 85.09) (end 175.26 86.36) (width 0.25) (layer "B.Cu") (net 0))
 (segment (start 137.16 71.12) (end 137.16 72.39) (width 0.25) (layer "B.Cu") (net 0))
 (segment (start 170.18 74.93) (end 170.18 78.74) (width 0.25) (layer "B.Cu") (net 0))
 (segment (start 157.48 66.04) (end 157.48 63.495) (width 0.25) (layer "B.Cu") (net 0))
 (segment (start 148.59 85.09) (end 149.86 86.36) (width 0.25) (layer "B.Cu") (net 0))
 (segment (start 165.1 71.12) (end 161.29 67.31) (width 0.25) (layer "B.Cu") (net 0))
 (segment (start 162.56 71.12) (end 159.385 67.945) (width 0.25) (layer "B.Cu") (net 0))
 (segment (start 170.18 60.955) (end 170.18 60.96) (width 0.25) (layer "B.Cu") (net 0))
 (segment (start 157.48 81.915) (end 157.48 86.36) (width 0.25) (layer "B.Cu") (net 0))
 (segment (start 157.48 68.58) (end 157.48 81.28) (width 0.25) (layer "B.Cu") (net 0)))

